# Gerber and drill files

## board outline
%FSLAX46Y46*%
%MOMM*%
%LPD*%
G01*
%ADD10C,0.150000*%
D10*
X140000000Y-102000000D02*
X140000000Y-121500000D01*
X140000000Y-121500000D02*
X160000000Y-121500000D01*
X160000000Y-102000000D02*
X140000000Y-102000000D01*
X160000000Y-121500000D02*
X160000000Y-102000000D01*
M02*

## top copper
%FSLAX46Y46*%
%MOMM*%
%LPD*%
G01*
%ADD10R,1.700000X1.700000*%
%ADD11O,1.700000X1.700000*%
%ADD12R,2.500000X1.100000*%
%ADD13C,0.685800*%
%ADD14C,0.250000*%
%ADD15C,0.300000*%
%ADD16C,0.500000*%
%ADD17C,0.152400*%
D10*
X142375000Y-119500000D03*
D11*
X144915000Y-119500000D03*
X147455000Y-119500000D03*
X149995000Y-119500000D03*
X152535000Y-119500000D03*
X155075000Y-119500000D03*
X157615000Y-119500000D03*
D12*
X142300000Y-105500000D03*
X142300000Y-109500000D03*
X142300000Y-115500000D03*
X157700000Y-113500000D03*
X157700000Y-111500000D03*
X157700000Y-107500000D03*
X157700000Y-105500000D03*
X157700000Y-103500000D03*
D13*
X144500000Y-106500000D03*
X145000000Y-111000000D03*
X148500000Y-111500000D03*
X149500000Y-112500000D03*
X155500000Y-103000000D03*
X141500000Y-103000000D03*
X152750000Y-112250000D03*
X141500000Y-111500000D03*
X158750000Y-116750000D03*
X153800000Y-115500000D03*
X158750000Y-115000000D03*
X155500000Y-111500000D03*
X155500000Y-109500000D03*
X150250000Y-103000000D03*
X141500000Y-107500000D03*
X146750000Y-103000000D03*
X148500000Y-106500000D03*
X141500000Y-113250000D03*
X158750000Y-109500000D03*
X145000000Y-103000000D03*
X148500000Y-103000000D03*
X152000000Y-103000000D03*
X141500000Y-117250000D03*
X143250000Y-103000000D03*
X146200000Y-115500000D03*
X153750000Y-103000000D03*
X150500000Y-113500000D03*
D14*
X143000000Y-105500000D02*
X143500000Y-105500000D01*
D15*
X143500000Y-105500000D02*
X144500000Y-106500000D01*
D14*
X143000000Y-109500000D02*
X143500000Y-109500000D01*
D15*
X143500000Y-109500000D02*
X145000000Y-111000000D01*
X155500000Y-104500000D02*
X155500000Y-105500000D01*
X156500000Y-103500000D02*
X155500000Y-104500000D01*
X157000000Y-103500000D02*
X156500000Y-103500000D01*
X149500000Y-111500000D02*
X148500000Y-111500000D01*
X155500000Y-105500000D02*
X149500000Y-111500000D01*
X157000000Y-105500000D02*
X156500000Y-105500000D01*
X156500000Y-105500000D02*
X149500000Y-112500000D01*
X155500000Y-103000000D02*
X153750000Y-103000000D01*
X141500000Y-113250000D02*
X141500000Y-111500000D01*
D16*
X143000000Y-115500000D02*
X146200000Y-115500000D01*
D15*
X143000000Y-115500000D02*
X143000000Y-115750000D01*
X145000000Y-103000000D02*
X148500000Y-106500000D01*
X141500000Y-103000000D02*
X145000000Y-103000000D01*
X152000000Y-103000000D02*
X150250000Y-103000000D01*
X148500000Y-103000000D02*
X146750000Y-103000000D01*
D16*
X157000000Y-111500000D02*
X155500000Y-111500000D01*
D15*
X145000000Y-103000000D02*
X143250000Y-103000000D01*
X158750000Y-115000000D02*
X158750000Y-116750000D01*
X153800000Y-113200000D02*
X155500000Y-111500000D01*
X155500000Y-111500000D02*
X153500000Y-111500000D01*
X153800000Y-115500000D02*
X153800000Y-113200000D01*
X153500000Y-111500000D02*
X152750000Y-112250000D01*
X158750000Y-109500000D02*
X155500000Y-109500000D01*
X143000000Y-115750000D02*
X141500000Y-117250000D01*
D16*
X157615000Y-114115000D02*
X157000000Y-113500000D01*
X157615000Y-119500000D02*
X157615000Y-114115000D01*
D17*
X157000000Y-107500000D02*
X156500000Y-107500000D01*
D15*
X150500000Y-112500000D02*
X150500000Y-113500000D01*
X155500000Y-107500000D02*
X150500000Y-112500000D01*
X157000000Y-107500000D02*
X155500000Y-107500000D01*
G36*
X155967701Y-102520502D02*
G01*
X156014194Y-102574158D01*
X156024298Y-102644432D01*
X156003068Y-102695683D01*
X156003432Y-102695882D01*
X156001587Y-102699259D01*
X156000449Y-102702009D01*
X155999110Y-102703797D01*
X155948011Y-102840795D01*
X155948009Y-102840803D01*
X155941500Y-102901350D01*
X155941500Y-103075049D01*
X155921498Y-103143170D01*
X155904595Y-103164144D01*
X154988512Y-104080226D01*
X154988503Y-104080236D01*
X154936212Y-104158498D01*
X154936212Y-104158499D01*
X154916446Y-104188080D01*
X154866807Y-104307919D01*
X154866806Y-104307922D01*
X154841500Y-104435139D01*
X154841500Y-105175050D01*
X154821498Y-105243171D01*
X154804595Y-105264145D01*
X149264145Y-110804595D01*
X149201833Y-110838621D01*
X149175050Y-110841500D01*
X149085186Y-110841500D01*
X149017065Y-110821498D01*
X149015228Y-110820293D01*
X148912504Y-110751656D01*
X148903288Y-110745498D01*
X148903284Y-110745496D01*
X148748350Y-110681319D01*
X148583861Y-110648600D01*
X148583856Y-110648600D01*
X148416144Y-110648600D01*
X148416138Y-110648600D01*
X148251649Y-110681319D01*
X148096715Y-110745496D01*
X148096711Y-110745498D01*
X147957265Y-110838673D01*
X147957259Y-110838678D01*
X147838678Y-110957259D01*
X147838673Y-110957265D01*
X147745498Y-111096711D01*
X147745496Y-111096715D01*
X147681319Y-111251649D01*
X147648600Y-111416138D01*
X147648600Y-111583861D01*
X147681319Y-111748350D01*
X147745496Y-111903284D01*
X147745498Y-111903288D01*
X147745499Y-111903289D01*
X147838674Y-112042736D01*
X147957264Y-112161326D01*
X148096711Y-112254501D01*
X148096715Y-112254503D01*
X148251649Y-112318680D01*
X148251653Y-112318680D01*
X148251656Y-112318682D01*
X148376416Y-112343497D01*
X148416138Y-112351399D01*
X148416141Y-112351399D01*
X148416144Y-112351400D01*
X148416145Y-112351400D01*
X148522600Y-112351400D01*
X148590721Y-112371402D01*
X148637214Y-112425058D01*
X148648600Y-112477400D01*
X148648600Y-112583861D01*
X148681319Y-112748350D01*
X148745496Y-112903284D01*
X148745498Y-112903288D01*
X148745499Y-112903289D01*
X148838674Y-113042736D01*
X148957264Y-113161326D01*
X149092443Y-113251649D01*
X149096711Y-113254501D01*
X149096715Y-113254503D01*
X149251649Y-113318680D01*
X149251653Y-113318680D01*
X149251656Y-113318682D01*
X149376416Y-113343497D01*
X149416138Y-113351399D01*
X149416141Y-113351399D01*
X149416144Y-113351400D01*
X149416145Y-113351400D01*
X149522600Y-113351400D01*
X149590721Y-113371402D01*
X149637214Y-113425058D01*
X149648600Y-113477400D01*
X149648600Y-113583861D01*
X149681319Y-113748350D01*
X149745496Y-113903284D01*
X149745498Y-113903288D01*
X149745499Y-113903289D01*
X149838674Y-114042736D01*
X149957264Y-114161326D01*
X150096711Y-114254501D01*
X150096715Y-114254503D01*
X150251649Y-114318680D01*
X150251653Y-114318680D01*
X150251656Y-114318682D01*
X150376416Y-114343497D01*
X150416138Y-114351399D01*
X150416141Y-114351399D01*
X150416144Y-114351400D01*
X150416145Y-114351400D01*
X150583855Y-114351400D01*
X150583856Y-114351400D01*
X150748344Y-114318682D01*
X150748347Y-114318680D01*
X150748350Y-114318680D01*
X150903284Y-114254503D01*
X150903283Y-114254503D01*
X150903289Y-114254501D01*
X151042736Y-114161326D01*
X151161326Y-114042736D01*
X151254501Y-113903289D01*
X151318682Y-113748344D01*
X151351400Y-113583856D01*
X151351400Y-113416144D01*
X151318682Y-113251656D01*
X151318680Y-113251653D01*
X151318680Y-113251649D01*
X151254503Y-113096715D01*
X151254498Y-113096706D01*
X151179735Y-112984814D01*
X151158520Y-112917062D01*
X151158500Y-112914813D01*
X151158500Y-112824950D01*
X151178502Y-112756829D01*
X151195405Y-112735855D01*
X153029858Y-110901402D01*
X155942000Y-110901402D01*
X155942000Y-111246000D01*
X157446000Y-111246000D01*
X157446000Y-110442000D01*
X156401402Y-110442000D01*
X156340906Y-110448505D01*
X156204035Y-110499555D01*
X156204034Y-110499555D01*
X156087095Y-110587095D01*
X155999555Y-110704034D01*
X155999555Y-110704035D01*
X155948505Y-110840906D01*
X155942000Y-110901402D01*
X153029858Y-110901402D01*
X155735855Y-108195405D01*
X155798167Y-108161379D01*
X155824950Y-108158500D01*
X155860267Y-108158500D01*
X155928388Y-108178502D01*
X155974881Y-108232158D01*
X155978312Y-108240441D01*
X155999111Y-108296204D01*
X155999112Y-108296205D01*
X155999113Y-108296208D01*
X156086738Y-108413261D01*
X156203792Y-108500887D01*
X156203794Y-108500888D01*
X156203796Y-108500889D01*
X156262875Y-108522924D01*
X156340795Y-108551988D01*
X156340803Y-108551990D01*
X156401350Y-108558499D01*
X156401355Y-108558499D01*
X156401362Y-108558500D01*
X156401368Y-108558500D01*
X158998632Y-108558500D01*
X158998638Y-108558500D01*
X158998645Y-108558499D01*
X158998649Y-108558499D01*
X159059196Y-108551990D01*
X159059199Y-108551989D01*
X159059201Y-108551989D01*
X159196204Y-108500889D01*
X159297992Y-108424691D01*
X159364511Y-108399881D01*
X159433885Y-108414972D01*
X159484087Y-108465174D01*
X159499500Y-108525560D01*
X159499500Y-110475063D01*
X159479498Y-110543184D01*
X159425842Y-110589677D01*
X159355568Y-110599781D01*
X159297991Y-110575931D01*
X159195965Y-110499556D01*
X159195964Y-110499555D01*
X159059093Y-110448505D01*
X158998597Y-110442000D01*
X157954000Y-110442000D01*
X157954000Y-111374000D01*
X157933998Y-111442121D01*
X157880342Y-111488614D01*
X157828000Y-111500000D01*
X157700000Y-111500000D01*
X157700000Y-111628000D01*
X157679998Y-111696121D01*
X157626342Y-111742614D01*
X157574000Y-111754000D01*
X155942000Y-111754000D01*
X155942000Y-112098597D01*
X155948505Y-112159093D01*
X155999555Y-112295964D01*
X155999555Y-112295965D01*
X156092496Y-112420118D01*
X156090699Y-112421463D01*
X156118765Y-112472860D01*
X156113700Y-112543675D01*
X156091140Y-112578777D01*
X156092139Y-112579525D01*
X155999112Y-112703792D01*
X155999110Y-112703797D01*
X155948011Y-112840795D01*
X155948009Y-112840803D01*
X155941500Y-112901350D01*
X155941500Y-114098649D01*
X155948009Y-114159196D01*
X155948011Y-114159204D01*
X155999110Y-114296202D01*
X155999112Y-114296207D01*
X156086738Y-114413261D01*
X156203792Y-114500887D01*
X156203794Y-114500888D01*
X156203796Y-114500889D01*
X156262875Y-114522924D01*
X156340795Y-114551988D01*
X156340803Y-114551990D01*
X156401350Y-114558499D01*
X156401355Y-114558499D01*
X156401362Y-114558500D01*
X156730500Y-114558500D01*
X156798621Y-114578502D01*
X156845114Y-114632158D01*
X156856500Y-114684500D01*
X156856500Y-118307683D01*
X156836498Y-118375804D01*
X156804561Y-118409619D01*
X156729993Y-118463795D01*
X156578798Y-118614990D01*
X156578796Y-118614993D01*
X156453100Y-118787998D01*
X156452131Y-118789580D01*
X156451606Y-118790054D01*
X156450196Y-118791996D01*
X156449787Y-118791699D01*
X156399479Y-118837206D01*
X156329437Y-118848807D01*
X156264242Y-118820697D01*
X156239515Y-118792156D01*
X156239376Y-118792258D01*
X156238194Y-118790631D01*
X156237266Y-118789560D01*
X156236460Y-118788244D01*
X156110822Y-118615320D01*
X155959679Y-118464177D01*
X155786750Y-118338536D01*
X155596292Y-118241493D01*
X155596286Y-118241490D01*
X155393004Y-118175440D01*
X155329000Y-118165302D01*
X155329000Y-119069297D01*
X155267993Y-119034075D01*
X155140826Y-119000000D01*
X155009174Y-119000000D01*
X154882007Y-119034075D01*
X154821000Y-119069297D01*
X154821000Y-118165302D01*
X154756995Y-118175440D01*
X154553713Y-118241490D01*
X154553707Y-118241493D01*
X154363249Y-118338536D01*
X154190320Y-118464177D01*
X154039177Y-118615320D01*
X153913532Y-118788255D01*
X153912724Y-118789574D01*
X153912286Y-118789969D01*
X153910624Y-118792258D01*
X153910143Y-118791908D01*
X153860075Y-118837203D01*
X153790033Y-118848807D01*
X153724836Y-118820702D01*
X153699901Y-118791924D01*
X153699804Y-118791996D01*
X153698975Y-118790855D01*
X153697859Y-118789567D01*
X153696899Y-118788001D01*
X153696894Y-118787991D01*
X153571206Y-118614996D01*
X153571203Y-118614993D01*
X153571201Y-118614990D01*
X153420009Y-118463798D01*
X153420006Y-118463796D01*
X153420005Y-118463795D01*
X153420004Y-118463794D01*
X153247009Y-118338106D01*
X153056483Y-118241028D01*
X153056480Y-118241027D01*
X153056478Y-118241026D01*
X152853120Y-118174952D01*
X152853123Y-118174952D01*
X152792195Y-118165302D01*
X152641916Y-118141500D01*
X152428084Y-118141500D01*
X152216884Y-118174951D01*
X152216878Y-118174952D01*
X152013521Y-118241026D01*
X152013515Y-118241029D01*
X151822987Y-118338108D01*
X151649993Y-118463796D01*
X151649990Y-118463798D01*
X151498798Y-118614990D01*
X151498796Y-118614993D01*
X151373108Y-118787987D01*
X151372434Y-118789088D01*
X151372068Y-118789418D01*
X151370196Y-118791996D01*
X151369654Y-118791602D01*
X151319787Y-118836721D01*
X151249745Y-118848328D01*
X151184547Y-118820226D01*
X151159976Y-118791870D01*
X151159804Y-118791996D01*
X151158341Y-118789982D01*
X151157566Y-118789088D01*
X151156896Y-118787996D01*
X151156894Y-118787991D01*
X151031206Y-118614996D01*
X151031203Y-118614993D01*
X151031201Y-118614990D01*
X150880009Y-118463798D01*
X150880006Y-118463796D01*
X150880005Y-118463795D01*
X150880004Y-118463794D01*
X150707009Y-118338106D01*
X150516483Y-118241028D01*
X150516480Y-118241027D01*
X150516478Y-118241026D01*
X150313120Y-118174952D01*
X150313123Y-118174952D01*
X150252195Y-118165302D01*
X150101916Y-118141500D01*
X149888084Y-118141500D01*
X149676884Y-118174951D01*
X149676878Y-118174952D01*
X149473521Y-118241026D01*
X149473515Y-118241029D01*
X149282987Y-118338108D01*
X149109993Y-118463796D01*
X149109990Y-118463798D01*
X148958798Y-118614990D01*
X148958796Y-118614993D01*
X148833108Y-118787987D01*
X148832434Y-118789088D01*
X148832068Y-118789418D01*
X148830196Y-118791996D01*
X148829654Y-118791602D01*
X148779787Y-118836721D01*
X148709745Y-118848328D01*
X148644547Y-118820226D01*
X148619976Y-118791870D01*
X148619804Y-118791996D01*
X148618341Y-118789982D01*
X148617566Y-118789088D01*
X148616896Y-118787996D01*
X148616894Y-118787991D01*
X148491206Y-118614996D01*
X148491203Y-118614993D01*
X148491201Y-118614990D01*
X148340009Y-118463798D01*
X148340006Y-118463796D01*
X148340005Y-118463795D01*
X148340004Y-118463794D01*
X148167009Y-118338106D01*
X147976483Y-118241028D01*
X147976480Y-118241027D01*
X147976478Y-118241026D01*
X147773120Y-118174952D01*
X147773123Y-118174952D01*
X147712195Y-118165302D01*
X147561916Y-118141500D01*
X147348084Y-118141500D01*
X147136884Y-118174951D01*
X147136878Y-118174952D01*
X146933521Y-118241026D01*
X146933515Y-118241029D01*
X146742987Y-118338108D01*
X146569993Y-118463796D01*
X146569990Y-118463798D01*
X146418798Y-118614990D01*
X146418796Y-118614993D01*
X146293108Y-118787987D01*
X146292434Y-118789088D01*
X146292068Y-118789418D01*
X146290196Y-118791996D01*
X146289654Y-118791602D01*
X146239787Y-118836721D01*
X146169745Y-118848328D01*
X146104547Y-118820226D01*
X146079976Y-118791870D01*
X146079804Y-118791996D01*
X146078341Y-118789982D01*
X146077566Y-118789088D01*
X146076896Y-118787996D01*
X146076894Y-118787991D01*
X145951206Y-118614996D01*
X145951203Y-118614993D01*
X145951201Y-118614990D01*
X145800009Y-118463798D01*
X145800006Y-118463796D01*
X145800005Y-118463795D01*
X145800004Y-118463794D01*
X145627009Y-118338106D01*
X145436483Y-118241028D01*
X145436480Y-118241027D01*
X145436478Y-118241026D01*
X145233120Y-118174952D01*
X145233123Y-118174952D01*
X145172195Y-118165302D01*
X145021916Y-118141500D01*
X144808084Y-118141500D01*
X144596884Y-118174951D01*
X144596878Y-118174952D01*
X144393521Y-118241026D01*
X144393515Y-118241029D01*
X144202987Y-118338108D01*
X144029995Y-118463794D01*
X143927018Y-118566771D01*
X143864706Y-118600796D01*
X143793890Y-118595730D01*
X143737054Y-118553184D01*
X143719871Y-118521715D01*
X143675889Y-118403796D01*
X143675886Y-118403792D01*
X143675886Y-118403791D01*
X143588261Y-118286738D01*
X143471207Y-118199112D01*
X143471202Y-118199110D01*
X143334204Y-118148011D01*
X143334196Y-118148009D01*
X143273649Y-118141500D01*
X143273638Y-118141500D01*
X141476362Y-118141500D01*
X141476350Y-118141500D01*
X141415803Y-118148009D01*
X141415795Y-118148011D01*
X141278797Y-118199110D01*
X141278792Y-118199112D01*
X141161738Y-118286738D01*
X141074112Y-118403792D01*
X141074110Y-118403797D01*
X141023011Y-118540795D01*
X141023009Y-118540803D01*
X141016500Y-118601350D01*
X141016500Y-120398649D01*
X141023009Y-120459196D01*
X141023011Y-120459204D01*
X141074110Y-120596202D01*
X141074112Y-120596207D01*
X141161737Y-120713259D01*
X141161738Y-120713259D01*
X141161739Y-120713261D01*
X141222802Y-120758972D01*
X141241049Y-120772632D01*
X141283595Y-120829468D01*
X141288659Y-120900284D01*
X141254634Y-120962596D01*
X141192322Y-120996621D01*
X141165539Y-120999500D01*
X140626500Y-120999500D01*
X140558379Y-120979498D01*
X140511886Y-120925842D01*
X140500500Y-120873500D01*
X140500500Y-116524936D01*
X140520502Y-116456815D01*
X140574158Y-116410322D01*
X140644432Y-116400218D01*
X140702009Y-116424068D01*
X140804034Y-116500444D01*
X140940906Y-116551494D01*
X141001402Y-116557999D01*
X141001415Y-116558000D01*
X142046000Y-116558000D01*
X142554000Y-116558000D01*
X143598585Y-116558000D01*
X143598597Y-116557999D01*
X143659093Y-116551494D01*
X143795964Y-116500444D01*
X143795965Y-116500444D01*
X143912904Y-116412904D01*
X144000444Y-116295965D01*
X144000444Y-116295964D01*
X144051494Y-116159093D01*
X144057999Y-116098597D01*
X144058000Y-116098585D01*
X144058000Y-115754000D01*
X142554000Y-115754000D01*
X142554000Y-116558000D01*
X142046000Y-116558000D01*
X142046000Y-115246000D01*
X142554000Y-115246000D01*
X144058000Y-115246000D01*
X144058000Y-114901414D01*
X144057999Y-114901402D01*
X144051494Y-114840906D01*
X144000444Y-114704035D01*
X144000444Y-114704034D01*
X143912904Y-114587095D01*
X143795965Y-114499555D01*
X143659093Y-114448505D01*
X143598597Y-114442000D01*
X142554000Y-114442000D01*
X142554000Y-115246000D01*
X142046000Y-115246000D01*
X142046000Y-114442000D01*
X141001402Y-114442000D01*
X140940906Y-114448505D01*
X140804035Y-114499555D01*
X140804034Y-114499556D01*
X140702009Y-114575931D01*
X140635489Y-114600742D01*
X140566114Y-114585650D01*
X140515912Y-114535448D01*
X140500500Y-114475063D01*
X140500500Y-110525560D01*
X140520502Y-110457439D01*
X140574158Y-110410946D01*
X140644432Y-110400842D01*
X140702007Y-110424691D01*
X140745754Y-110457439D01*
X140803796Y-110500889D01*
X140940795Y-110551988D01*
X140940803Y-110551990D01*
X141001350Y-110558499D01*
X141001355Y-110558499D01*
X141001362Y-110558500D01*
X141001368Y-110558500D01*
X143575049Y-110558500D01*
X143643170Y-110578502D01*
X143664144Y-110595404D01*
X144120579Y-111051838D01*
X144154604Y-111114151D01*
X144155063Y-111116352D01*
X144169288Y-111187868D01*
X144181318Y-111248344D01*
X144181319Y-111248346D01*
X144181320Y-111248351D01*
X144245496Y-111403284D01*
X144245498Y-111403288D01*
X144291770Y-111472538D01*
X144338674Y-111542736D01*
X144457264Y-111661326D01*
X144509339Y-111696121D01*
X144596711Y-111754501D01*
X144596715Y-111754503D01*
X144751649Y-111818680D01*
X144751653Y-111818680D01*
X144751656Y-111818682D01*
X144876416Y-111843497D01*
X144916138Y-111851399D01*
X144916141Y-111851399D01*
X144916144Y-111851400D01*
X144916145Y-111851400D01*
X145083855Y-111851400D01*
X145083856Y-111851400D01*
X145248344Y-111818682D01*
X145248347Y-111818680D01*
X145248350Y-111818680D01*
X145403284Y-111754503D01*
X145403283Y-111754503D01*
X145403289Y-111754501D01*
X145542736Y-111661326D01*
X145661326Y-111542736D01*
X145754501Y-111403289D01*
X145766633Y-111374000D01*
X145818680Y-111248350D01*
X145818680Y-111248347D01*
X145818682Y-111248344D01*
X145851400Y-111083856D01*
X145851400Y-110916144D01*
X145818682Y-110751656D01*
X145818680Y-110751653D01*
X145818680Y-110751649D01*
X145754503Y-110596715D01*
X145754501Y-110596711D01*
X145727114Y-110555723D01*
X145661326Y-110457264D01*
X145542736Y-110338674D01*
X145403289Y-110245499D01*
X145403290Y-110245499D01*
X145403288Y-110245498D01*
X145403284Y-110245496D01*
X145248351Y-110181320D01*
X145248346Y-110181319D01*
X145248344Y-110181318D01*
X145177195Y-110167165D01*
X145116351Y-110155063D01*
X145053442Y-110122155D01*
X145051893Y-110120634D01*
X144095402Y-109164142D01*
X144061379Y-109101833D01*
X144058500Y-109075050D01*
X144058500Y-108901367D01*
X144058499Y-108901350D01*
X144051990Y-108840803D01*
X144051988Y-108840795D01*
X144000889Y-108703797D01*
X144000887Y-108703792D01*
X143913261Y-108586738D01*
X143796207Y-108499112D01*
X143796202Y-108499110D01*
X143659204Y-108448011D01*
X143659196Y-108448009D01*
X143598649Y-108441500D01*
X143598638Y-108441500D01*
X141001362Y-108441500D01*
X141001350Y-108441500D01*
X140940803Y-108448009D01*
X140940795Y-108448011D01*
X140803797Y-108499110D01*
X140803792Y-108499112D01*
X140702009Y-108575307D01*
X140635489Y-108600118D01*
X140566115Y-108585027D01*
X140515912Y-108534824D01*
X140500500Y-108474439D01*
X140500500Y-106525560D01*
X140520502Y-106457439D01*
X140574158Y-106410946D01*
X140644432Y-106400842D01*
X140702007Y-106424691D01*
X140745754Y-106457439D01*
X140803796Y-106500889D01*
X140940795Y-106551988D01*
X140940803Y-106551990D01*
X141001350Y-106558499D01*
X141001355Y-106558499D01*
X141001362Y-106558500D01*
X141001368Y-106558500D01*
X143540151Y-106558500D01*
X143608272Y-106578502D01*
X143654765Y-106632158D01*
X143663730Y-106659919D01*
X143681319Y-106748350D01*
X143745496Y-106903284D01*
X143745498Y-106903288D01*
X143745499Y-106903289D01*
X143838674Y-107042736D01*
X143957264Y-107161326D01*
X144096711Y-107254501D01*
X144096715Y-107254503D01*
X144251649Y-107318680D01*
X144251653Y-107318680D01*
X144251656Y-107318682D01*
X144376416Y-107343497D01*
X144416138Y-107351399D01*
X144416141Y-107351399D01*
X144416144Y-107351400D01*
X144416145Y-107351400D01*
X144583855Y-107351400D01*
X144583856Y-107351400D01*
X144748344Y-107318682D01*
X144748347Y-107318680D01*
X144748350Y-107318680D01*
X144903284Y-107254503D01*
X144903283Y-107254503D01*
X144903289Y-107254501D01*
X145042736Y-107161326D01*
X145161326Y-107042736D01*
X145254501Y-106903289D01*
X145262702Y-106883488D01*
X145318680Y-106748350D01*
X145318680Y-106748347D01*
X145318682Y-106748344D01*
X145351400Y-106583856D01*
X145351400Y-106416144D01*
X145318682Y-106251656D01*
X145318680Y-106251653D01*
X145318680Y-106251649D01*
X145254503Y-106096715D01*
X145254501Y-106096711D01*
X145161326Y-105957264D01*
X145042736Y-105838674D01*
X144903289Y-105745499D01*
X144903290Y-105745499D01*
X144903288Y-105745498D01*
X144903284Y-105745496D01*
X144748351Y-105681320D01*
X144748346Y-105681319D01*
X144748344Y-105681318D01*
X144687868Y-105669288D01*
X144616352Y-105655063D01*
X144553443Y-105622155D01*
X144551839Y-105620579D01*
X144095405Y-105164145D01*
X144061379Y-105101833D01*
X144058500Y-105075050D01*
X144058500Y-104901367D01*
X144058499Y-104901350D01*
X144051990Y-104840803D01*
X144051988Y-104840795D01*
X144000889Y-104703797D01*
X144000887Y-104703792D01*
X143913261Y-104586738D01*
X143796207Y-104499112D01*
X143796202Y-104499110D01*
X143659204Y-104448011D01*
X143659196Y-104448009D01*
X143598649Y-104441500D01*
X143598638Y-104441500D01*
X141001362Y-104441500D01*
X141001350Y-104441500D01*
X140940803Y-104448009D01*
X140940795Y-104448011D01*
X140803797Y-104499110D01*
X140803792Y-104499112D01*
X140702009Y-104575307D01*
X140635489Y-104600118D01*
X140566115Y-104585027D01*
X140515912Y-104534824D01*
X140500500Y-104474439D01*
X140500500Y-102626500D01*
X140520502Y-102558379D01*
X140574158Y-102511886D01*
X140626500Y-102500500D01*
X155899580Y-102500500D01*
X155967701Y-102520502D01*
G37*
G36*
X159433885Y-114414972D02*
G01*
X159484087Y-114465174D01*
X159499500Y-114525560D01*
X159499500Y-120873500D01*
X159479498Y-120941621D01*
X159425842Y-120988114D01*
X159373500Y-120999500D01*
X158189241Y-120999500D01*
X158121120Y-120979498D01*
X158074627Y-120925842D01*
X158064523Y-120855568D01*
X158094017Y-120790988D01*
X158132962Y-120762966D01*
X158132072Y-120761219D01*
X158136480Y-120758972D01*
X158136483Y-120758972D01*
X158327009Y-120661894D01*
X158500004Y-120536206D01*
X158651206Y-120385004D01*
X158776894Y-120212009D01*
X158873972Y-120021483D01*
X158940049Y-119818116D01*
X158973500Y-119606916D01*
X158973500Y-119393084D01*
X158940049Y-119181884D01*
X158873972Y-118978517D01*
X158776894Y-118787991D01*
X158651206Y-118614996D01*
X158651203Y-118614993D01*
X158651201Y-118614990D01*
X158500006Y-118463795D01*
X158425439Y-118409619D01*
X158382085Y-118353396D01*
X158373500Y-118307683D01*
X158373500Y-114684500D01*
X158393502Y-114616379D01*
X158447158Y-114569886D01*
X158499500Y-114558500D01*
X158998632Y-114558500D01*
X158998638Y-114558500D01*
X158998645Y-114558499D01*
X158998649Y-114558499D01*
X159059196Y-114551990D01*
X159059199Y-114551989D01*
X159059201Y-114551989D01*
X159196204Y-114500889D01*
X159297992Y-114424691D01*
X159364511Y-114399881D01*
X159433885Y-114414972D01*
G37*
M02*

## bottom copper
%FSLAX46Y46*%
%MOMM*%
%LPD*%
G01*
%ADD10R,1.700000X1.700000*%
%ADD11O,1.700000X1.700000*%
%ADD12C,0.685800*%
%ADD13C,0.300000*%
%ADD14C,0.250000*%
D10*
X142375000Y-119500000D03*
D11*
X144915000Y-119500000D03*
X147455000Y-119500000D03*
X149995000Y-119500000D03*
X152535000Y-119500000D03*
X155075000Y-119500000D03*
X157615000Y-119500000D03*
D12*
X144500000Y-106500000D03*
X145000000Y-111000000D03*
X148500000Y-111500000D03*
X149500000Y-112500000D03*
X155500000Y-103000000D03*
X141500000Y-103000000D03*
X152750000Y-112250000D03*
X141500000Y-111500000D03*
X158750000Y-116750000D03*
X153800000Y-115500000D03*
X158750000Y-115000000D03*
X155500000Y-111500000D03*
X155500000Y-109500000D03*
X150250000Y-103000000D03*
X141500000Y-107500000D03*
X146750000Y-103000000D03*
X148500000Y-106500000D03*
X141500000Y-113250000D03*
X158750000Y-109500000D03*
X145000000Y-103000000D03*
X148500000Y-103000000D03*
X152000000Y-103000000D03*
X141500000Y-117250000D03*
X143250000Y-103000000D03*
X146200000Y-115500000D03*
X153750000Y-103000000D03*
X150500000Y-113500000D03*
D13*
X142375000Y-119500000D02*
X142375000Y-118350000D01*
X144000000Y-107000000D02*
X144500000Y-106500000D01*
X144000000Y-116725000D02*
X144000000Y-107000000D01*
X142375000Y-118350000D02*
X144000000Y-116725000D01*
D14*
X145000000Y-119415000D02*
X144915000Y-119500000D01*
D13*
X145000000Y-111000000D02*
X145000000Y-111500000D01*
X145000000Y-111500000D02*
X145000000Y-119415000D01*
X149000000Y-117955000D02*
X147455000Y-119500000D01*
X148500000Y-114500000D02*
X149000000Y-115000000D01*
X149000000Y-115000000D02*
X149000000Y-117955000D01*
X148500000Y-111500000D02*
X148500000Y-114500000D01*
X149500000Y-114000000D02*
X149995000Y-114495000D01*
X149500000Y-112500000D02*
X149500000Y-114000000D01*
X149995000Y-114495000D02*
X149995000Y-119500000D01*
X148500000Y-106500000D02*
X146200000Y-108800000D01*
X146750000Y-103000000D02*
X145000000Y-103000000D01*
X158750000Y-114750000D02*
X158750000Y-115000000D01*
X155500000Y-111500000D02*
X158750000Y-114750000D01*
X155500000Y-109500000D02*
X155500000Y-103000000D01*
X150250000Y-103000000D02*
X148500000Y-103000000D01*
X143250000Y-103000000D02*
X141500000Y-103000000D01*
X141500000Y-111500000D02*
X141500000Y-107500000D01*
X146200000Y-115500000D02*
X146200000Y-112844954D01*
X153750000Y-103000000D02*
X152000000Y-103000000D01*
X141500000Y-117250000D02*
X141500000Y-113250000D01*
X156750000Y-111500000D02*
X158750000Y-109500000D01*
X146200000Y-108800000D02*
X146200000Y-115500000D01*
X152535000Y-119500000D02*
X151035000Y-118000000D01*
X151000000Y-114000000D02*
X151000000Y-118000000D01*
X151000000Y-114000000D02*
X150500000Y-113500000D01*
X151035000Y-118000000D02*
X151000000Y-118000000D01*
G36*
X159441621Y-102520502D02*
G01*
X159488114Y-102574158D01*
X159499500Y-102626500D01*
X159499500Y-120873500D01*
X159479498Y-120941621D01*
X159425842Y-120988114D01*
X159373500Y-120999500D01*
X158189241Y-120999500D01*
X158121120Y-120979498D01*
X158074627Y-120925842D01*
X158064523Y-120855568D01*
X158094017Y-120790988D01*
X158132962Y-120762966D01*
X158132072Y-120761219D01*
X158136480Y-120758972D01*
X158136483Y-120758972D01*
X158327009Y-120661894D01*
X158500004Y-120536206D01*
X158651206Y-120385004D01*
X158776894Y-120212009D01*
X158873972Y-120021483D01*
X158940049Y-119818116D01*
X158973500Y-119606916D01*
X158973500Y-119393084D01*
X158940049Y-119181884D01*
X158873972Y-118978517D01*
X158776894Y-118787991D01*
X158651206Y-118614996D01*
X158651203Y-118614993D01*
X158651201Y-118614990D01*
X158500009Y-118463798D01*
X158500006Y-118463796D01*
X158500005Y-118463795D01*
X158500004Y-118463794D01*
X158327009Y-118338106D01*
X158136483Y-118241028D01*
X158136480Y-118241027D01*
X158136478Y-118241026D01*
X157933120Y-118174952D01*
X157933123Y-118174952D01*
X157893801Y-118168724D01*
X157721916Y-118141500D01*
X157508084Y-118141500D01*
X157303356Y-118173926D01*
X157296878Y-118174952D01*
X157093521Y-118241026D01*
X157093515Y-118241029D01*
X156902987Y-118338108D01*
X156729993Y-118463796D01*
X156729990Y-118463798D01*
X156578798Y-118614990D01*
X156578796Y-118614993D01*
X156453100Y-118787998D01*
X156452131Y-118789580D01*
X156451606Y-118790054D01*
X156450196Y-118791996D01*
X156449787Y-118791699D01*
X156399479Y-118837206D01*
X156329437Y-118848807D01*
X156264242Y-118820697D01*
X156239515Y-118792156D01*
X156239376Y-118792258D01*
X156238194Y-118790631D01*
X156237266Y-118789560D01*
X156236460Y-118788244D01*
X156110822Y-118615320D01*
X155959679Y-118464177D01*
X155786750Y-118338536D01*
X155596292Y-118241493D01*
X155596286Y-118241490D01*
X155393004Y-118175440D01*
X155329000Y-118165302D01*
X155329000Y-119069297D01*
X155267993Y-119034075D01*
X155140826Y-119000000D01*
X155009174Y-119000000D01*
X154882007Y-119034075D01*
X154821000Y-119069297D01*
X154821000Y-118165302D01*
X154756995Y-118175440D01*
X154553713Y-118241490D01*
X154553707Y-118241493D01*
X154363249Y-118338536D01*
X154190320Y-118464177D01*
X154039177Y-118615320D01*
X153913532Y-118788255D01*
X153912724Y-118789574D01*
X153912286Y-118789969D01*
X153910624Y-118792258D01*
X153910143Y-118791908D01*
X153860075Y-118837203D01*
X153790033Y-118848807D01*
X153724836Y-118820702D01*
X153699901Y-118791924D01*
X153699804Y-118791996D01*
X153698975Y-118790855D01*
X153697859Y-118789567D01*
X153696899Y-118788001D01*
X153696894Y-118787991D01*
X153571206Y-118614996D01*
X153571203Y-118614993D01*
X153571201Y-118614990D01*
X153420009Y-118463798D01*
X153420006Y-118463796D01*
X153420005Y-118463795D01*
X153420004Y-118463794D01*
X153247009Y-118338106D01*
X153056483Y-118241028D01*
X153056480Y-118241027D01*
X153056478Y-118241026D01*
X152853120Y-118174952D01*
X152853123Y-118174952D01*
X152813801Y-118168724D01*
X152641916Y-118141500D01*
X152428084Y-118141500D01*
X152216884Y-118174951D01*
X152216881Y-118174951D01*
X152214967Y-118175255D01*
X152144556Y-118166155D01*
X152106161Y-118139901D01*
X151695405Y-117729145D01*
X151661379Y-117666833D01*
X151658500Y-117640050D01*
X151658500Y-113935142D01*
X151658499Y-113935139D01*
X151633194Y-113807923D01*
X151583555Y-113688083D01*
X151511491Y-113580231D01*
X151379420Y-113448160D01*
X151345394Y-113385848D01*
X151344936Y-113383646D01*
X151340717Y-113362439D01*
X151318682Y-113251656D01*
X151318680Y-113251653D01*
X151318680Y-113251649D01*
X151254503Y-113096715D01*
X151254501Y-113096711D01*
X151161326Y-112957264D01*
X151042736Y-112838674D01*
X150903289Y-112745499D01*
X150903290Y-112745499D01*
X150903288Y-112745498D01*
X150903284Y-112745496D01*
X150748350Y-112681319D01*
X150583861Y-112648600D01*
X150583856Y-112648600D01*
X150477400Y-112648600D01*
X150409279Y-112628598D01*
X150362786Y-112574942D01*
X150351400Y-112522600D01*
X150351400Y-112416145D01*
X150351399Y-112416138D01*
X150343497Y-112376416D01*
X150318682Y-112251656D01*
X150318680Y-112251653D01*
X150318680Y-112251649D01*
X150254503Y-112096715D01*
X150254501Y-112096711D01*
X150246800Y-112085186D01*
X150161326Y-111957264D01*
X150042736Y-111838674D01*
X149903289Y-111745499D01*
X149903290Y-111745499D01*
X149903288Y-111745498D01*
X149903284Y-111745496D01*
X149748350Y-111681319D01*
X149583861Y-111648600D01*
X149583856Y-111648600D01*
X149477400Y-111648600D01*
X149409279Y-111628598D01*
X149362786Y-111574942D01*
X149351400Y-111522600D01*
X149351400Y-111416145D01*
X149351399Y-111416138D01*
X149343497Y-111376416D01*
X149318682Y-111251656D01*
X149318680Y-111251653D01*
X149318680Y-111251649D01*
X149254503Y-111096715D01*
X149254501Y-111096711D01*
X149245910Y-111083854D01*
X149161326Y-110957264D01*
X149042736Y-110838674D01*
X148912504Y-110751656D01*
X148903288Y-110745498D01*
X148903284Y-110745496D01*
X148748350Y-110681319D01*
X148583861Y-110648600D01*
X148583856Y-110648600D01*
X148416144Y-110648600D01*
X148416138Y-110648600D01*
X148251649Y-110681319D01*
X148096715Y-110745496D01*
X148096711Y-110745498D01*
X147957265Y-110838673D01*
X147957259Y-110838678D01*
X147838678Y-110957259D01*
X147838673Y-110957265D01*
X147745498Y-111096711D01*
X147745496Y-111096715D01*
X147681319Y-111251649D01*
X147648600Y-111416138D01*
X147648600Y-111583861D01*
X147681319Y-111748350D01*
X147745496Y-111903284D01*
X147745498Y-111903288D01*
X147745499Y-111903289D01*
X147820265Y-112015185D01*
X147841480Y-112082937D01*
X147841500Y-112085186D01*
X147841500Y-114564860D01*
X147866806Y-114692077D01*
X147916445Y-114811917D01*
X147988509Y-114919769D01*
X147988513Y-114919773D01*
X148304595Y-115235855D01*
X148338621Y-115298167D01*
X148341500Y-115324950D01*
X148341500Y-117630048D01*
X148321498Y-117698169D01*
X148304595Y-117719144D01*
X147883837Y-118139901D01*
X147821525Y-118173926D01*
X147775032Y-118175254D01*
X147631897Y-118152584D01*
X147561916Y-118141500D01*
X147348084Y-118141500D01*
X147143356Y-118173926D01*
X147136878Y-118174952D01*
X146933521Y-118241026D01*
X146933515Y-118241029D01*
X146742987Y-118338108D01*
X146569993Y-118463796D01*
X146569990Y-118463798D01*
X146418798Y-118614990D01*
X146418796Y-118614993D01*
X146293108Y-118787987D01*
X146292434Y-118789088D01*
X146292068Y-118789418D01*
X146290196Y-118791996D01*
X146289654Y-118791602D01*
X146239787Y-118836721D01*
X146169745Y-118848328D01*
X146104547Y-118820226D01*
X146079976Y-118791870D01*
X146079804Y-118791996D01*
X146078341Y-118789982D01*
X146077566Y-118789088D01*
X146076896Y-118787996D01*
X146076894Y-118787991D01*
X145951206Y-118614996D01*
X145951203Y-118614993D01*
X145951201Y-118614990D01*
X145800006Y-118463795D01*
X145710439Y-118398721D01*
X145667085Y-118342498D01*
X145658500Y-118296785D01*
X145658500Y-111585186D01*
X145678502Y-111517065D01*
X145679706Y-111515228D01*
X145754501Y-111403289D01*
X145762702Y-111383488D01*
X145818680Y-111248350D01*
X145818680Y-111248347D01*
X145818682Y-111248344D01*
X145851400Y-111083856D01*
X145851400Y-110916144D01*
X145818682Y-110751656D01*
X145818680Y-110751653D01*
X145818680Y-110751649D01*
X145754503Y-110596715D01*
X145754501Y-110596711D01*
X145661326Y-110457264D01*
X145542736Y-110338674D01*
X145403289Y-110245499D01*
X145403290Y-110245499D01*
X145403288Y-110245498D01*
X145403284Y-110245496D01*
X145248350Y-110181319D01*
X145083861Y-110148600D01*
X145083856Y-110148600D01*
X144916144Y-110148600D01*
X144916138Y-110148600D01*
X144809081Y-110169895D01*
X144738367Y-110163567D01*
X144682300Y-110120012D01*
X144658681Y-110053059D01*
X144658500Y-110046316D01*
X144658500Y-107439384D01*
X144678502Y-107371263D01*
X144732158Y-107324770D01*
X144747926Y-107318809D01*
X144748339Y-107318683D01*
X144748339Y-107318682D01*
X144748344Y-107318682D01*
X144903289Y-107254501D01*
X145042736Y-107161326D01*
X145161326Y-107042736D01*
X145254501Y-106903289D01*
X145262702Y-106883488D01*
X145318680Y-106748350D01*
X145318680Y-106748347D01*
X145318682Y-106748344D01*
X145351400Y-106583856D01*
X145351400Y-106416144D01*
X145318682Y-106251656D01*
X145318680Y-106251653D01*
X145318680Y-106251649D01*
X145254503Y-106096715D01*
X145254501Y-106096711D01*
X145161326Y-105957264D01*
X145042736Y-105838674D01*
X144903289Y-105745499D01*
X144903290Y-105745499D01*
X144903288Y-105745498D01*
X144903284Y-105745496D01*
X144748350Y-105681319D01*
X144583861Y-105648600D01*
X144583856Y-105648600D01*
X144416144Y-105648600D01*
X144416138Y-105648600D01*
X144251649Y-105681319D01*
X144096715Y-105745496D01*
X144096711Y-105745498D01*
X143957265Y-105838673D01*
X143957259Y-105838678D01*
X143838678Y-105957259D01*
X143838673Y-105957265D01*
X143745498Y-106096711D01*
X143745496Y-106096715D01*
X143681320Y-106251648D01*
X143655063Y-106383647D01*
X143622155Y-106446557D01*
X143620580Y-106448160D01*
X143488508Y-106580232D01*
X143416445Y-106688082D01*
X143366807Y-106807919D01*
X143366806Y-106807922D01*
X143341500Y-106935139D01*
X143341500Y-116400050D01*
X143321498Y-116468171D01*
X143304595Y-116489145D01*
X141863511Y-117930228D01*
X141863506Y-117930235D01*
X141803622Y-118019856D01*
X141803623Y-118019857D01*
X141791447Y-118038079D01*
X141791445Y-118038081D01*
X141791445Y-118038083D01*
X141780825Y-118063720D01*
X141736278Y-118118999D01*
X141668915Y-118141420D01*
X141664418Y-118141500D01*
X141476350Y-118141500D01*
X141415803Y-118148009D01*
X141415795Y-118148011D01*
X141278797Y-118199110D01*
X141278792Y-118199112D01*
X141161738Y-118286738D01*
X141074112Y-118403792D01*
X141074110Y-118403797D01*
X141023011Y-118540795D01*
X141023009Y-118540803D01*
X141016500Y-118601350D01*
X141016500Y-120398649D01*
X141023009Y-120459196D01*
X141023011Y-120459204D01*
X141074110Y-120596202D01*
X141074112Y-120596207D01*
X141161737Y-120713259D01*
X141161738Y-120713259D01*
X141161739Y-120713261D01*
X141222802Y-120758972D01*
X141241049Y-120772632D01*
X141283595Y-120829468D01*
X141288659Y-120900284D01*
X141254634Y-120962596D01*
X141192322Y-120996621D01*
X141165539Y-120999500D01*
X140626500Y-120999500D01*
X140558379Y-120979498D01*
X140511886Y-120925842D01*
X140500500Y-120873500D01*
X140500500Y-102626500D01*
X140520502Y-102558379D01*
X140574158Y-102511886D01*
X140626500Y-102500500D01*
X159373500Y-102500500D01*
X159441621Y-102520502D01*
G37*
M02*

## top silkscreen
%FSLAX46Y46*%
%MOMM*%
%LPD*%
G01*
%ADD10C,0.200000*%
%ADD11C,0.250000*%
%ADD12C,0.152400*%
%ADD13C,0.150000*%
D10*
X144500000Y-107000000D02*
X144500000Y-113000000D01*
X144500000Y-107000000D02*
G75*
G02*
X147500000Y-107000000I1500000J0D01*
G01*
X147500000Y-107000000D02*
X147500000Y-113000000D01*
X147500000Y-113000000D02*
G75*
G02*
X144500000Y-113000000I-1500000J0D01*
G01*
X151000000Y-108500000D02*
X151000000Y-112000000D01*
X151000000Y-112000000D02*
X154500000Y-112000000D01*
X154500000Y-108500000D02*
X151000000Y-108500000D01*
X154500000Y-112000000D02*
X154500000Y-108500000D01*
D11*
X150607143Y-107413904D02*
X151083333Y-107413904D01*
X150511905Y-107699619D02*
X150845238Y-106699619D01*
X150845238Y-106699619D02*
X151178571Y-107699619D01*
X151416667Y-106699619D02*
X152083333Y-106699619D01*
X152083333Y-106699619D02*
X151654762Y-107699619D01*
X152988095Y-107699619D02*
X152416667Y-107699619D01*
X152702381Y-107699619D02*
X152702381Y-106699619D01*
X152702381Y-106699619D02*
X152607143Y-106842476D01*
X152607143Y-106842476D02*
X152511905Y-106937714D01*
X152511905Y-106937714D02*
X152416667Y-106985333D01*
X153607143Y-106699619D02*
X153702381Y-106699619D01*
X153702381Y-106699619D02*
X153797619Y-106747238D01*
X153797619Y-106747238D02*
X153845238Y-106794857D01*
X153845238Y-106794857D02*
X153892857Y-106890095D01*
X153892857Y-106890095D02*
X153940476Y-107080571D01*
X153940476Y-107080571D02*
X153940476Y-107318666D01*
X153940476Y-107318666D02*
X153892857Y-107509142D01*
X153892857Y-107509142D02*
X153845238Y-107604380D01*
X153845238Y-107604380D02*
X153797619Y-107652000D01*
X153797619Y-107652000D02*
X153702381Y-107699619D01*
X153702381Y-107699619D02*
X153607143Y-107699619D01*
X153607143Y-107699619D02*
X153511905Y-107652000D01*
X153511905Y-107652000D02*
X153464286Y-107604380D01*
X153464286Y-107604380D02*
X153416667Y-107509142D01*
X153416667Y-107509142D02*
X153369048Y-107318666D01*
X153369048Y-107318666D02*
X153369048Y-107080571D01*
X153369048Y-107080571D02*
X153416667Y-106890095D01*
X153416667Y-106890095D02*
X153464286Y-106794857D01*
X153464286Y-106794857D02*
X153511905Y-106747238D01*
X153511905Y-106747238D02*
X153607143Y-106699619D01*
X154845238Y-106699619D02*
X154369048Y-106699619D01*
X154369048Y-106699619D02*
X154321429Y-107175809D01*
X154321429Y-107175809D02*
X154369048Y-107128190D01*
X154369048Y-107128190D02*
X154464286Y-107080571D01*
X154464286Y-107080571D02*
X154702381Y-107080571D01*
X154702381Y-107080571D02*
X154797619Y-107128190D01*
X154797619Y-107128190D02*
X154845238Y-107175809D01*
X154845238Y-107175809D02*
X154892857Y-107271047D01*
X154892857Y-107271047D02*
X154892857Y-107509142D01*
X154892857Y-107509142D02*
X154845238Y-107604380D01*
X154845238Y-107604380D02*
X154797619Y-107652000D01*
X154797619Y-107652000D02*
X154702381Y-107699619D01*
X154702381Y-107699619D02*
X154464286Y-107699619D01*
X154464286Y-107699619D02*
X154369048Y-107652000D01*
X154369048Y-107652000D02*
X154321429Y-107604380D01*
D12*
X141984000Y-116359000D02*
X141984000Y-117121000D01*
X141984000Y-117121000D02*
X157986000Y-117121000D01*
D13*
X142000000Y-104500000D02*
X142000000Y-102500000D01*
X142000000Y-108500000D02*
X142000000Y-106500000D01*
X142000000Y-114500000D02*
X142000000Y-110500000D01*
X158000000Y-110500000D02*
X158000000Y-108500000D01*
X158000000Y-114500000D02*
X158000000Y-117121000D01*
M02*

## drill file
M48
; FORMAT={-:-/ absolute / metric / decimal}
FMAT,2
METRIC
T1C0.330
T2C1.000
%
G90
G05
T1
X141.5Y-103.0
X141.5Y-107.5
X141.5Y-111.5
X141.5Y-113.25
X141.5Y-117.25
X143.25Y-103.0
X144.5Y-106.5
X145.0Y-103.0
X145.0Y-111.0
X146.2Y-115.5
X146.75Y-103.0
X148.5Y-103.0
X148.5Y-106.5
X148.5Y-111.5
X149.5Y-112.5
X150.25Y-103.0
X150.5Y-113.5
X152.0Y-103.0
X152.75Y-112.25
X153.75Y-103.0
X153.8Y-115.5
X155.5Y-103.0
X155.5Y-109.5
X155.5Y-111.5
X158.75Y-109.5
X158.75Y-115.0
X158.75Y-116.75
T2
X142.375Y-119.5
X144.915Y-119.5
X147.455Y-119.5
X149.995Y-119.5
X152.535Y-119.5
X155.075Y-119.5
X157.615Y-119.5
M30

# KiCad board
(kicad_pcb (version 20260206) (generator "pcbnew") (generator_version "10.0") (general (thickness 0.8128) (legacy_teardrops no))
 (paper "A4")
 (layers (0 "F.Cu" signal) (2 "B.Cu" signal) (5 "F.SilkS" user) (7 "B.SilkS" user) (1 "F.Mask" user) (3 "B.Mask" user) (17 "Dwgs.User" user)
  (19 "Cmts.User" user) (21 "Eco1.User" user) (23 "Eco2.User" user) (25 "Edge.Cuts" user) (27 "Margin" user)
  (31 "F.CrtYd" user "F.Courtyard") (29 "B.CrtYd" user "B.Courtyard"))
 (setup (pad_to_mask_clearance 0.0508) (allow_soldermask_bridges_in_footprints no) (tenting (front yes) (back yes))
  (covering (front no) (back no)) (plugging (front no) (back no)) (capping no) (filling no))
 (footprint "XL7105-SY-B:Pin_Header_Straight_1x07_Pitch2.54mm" (layer "F.Cu") (at 142.375 119.5 90)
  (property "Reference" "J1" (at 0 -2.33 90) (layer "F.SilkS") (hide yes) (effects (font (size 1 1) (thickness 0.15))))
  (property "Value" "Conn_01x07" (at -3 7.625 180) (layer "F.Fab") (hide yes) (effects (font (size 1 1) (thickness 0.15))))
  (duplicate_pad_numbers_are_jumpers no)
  (pad "1" thru_hole rect (at 0 0 90) (size 1.7 1.7) (drill 1) (layers "*.Cu" "*.Mask") (remove_unused_layers no) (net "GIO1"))
  (pad "2" thru_hole oval (at 0 2.54 90) (size 1.7 1.7) (drill 1) (layers "*.Cu" "*.Mask") (remove_unused_layers no) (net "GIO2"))
  (pad "3" thru_hole oval (at 0 5.08 90) (size 1.7 1.7) (drill 1) (layers "*.Cu" "*.Mask") (remove_unused_layers no) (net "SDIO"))
  (pad "4" thru_hole oval (at 0 7.62 90) (size 1.7 1.7) (drill 1) (layers "*.Cu" "*.Mask") (remove_unused_layers no) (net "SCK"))
  (pad "5" thru_hole oval (at 0 10.16 90) (size 1.7 1.7) (drill 1) (layers "*.Cu" "*.Mask") (remove_unused_layers no) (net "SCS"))
  (pad "6" thru_hole oval (at 0 12.7 90) (size 1.7 1.7) (drill 1) (layers "*.Cu" "*.Mask") (remove_unused_layers no) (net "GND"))
  (pad "7" thru_hole oval (at 0 15.24 90) (size 1.7 1.7) (drill 1) (layers "*.Cu" "*.Mask") (remove_unused_layers no) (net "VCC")))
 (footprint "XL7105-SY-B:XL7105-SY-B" (layer "F.Cu") (at 143 103.5)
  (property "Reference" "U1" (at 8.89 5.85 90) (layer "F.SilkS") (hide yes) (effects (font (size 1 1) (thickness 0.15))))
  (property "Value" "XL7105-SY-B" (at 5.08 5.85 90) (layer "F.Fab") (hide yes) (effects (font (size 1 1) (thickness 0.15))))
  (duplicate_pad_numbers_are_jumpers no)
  (fp_line (start -1.016 12.859) (end -1.016 13.621) (stroke (width 0.1524) (type solid)) (layer "F.SilkS"))
  (fp_line (start -1.016 13.621) (end 14.986 13.621) (stroke (width 0.1524) (type solid)) (layer "F.SilkS"))
  (fp_line (start -1 1) (end -1 -1) (stroke (width 0.15) (type solid)) (layer "F.SilkS"))
  (fp_line (start -1 5) (end -1 3) (stroke (width 0.15) (type solid)) (layer "F.SilkS"))
  (fp_line (start -1 11) (end -1 7) (stroke (width 0.15) (type solid)) (layer "F.SilkS"))
  (fp_line (start 15 7) (end 15 5) (stroke (width 0.15) (type solid)) (layer "F.SilkS"))
  (fp_line (start 15 11) (end 15 13.621) (stroke (width 0.15) (type solid)) (layer "F.SilkS"))
  (pad "2" smd rect (at 0 2) (size 2.5 1.1) (drill (offset -0.7 0)) (layers "F.Cu" "F.Mask") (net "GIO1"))
  (pad "4" smd rect (at 0 6) (size 2.5 1.1) (drill (offset -0.7 0)) (layers "F.Cu" "F.Mask") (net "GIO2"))
  (pad "7" smd rect (at 0 12) (size 2.5 1.1) (drill (offset -0.7 0)) (layers "F.Cu" "F.Mask") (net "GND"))
  (pad "9" smd rect (at 14 10) (size 2.5 1.1) (drill (offset 0.7 0)) (layers "F.Cu" "F.Mask") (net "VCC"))
  (pad "10" smd rect (at 14 8) (size 2.5 1.1) (drill (offset 0.7 0)) (layers "F.Cu" "F.Mask") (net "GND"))
  (pad "12" smd rect (at 14 4) (size 2.5 1.1) (drill (offset 0.7 0)) (layers "F.Cu" "F.Mask") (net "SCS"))
  (pad "13" smd rect (at 14 2) (size 2.5 1.1) (drill (offset 0.7 0)) (layers "F.Cu" "F.Mask") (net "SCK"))
  (pad "14" smd rect (at 14 0) (size 2.5 1.1) (drill (offset 0.7 0)) (layers "F.Cu" "F.Mask") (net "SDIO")))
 (gr_line (start 144.5 107) (end 144.5 113) (stroke (width 0.2) (type solid)) (layer "F.SilkS"))
 (gr_arc (start 144.5 107) (mid 146 105.5) (end 147.5 107) (stroke (width 0.2) (type solid)) (layer "F.SilkS"))
 (gr_line (start 147.5 107) (end 147.5 113) (stroke (width 0.2) (type solid)) (layer "F.SilkS"))
 (gr_arc (start 147.5 113) (mid 146 114.5) (end 144.5 113) (stroke (width 0.2) (type solid)) (layer "F.SilkS"))
 (gr_line (start 151 108.5) (end 151 112) (stroke (width 0.2) (type solid)) (layer "F.SilkS"))
 (gr_line (start 151 112) (end 154.5 112) (stroke (width 0.2) (type solid)) (layer "F.SilkS"))
 (gr_line (start 154.5 108.5) (end 151 108.5) (stroke (width 0.2) (type solid)) (layer "F.SilkS"))
 (gr_line (start 154.5 112) (end 154.5 108.5) (stroke (width 0.2) (type solid)) (layer "F.SilkS"))
 (gr_line (start 140 102) (end 140 121.5) (stroke (width 0.15) (type solid)) (layer "Edge.Cuts"))
 (gr_line (start 140 121.5) (end 160 121.5) (stroke (width 0.15) (type solid)) (layer "Edge.Cuts"))
 (gr_line (start 160 102) (end 140 102) (stroke (width 0.15) (type solid)) (layer "Edge.Cuts"))
 (gr_line (start 160 121.5) (end 160 102) (stroke (width 0.15) (type solid)) (layer "Edge.Cuts"))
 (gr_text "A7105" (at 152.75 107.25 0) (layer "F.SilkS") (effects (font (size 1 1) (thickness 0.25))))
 (segment (start 143 105.5) (end 143.5 105.5) (width 0.25) (layer "F.Cu") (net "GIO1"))
 (segment (start 143.5 105.5) (end 144.5 106.5) (width 0.3) (layer "F.Cu") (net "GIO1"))
 (via (at 144.5 106.5) (size 0.6858) (drill 0.3302) (layers "F.Cu" "B.Cu") (capping no) (covering (front no) (back no))
  (plugging (front no) (back no)) (filling no) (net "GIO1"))
 (segment (start 142.375 119.5) (end 142.375 118.35) (width 0.3) (layer "B.Cu") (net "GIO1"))
 (segment (start 144 107) (end 144.5 106.5) (width 0.3) (layer "B.Cu") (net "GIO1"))
 (segment (start 144 116.725) (end 144 107) (width 0.3) (layer "B.Cu") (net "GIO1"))
 (segment (start 142.375 118.35) (end 144 116.725) (width 0.3) (layer "B.Cu") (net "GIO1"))
 (segment (start 143 109.5) (end 143.5 109.5) (width 0.25) (layer "F.Cu") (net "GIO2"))
 (segment (start 143.5 109.5) (end 145 111) (width 0.3) (layer "F.Cu") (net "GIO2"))
 (via (at 145 111) (size 0.6858) (drill 0.3302) (layers "F.Cu" "B.Cu") (capping no) (covering (front no) (back no))
  (plugging (front no) (back no)) (filling no) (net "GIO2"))
 (segment (start 145 119.415) (end 144.915 119.5) (width 0.25) (layer "B.Cu") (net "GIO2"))
 (segment (start 145 111) (end 145 111.5) (width 0.3) (layer "B.Cu") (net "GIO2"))
 (segment (start 145 111.5) (end 145 119.415) (width 0.3) (layer "B.Cu") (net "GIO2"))
 (segment (start 155.5 104.5) (end 155.5 105.5) (width 0.3) (layer "F.Cu") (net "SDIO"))
 (segment (start 156.5 103.5) (end 155.5 104.5) (width 0.3) (layer "F.Cu") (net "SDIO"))
 (segment (start 157 103.5) (end 156.5 103.5) (width 0.3) (layer "F.Cu") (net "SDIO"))
 (segment (start 149.5 111.5) (end 148.5 111.5) (width 0.3) (layer "F.Cu") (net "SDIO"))
 (segment (start 155.5 105.5) (end 149.5 111.5) (width 0.3) (layer "F.Cu") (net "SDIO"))
 (via (at 148.5 111.5) (size 0.6858) (drill 0.3302) (layers "F.Cu" "B.Cu") (capping no) (covering (front no) (back no))
  (plugging (front no) (back no)) (filling no) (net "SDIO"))
 (segment (start 149 117.955) (end 147.455 119.5) (width 0.3) (layer "B.Cu") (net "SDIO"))
 (segment (start 148.5 114.5) (end 149 115) (width 0.3) (layer "B.Cu") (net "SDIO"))
 (segment (start 149 115) (end 149 117.955) (width 0.3) (layer "B.Cu") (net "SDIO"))
 (segment (start 148.5 111.5) (end 148.5 114.5) (width 0.3) (layer "B.Cu") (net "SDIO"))
 (segment (start 157 105.5) (end 156.5 105.5) (width 0.3) (layer "F.Cu") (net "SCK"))
 (segment (start 156.5 105.5) (end 149.5 112.5) (width 0.3) (layer "F.Cu") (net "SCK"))
 (via (at 149.5 112.5) (size 0.6858) (drill 0.3302) (layers "F.Cu" "B.Cu") (capping no) (covering (front no) (back no))
  (plugging (front no) (back no)) (filling no) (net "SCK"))
 (segment (start 149.5 114) (end 149.995 114.495) (width 0.3) (layer "B.Cu") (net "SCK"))
 (segment (start 149.5 112.5) (end 149.5 114) (width 0.3) (layer "B.Cu") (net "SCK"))
 (segment (start 149.995 114.495) (end 149.995 119.5) (width 0.3) (layer "B.Cu") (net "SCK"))
 (segment (start 155.5 103) (end 153.75 103) (width 0.3) (layer "F.Cu") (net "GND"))
 (segment (start 141.5 113.25) (end 141.5 111.5) (width 0.3) (layer "F.Cu") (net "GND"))
 (segment (start 143 115.5) (end 146.2 115.5) (width 0.5) (layer "F.Cu") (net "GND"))
 (segment (start 143 115.5) (end 143 115.75) (width 0.3) (layer "F.Cu") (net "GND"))
 (segment (start 145 103) (end 148.5 106.5) (width 0.3) (layer "F.Cu") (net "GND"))
 (segment (start 141.5 103) (end 145 103) (width 0.3) (layer "F.Cu") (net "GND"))
 (segment (start 152 103) (end 150.25 103) (width 0.3) (layer "F.Cu") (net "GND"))
 (segment (start 148.5 103) (end 146.75 103) (width 0.3) (layer "F.Cu") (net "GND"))
 (segment (start 157 111.5) (end 155.5 111.5) (width 0.5) (layer "F.Cu") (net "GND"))
 (segment (start 145 103) (end 143.25 103) (width 0.3) (layer "F.Cu") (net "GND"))
 (segment (start 158.75 115) (end 158.75 116.75) (width 0.3) (layer "F.Cu") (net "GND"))
 (segment (start 153.8 113.2) (end 155.5 111.5) (width 0.3) (layer "F.Cu") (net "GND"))
 (segment (start 155.5 111.5) (end 153.5 111.5) (width 0.3) (layer "F.Cu") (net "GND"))
 (segment (start 153.8 115.5) (end 153.8 113.2) (width 0.3) (layer "F.Cu") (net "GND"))
 (segment (start 153.5 111.5) (end 152.75 112.25) (width 0.3) (layer "F.Cu") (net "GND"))
 (segment (start 158.75 109.5) (end 155.5 109.5) (width 0.3) (layer "F.Cu") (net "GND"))
 (segment (start 143 115.75) (end 141.5 117.25) (width 0.3) (layer "F.Cu") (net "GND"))
 (via (at 155.5 103) (size 0.6858) (drill 0.3302) (layers "F.Cu" "B.Cu") (capping no) (covering (front no) (back no))
  (plugging (front no) (back no)) (filling no) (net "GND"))
 (via (at 141.5 103) (size 0.6858) (drill 0.3302) (layers "F.Cu" "B.Cu") (capping no) (covering (front no) (back no))
  (plugging (front no) (back no)) (filling no) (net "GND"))
 (via (at 152.75 112.25) (size 0.6858) (drill 0.3302) (layers "F.Cu" "B.Cu") (capping no) (covering (front no) (back no))
  (plugging (front no) (back no)) (filling no) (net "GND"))
 (via (at 141.5 111.5) (size 0.6858) (drill 0.3302) (layers "F.Cu" "B.Cu") (capping no) (covering (front no) (back no))
  (plugging (front no) (back no)) (filling no) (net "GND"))
 (via (at 158.75 116.75) (size 0.6858) (drill 0.3302) (layers "F.Cu" "B.Cu") (capping no) (covering (front no) (back no))
  (plugging (front no) (back no)) (filling no) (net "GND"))
 (via (at 153.8 115.5) (size 0.6858) (drill 0.3302) (layers "F.Cu" "B.Cu") (capping no) (covering (front no) (back no))
  (plugging (front no) (back no)) (filling no) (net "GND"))
 (via (at 158.75 115) (size 0.6858) (drill 0.3302) (layers "F.Cu" "B.Cu") (capping no) (covering (front no) (back no))
  (plugging (front no) (back no)) (filling no) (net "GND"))
 (via (at 155.5 111.5) (size 0.6858) (drill 0.3302) (layers "F.Cu" "B.Cu") (capping no) (covering (front no) (back no))
  (plugging (front no) (back no)) (filling no) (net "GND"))
 (via (at 155.5 109.5) (size 0.6858) (drill 0.3302) (layers "F.Cu" "B.Cu") (capping no) (covering (front no) (back no))
  (plugging (front no) (back no)) (filling no) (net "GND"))
 (via (at 150.25 103) (size 0.6858) (drill 0.3302) (layers "F.Cu" "B.Cu") (capping no) (covering (front no) (back no))
  (plugging (front no) (back no)) (filling no) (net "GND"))
 (via (at 141.5 107.5) (size 0.6858) (drill 0.3302) (layers "F.Cu" "B.Cu") (capping no) (covering (front no) (back no))
  (plugging (front no) (back no)) (filling no) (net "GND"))
 (via (at 146.75 103) (size 0.6858) (drill 0.3302) (layers "F.Cu" "B.Cu") (capping no) (covering (front no) (back no))
  (plugging (front no) (back no)) (filling no) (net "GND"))
 (via (at 148.5 106.5) (size 0.6858) (drill 0.3302) (layers "F.Cu" "B.Cu") (capping no) (covering (front no) (back no))
  (plugging (front no) (back no)) (filling no) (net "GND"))
 (via (at 141.5 113.25) (size 0.6858) (drill 0.3302) (layers "F.Cu" "B.Cu") (capping no) (covering (front no) (back no))
  (plugging (front no) (back no)) (filling no) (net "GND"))
 (via (at 158.75 109.5) (size 0.6858) (drill 0.3302) (layers "F.Cu" "B.Cu") (capping no) (covering (front no) (back no))
  (plugging (front no) (back no)) (filling no) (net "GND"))
 (via (at 145 103) (size 0.6858) (drill 0.3302) (layers "F.Cu" "B.Cu") (capping no) (covering (front no) (back no))
  (plugging (front no) (back no)) (filling no) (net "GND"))
 (via (at 148.5 103) (size 0.6858) (drill 0.3302) (layers "F.Cu" "B.Cu") (capping no) (covering (front no) (back no))
  (plugging (front no) (back no)) (filling no) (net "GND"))
 (via (at 152 103) (size 0.6858) (drill 0.3302) (layers "F.Cu" "B.Cu") (capping no) (covering (front no) (back no))
  (plugging (front no) (back no)) (filling no) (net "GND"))
 (via (at 141.5 117.25) (size 0.6858) (drill 0.3302) (layers "F.Cu" "B.Cu") (capping no) (covering (front no) (back no))
  (plugging (front no) (back no)) (filling no) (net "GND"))
 (via (at 143.25 103) (size 0.6858) (drill 0.3302) (layers "F.Cu" "B.Cu") (capping no) (covering (front no) (back no))
  (plugging (front no) (back no)) (filling no) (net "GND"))
 (via (at 146.2 115.5) (size 0.6858) (drill 0.3302) (layers "F.Cu" "B.Cu") (capping no) (covering (front no) (back no))
  (plugging (front no) (back no)) (filling no) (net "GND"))
 (via (at 153.75 103) (size 0.6858) (drill 0.3302) (layers "F.Cu" "B.Cu") (capping no) (covering (front no) (back no))
  (plugging (front no) (back no)) (filling no) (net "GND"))
 (segment (start 148.5 106.5) (end 146.2 108.8) (width 0.3) (layer "B.Cu") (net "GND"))
 (segment (start 146.75 103) (end 145 103) (width 0.3) (layer "B.Cu") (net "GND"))
 (segment (start 158.75 114.75) (end 158.75 115) (width 0.3) (layer "B.Cu") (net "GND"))
 (segment (start 155.5 111.5) (end 158.75 114.75) (width 0.3) (layer "B.Cu") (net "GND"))
 (segment (start 155.5 109.5) (end 155.5 103) (width 0.3) (layer "B.Cu") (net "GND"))
 (segment (start 150.25 103) (end 148.5 103) (width 0.3) (layer "B.Cu") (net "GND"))
 (segment (start 143.25 103) (end 141.5 103) (width 0.3) (layer "B.Cu") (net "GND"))
 (segment (start 141.5 111.5) (end 141.5 107.5) (width 0.3) (layer "B.Cu") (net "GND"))
 (segment (start 146.2 115.5) (end 146.2 112.844954) (width 0.3) (layer "B.Cu") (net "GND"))
 (segment (start 153.75 103) (end 152 103) (width 0.3) (layer "B.Cu") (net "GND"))
 (segment (start 141.5 117.25) (end 141.5 113.25) (width 0.3) (layer "B.Cu") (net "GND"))
 (segment (start 156.75 111.5) (end 158.75 109.5) (width 0.3) (layer "B.Cu") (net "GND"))
 (segment (start 146.2 108.8) (end 146.2 115.5) (width 0.3) (layer "B.Cu") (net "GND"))
 (segment (start 157.615 114.115) (end 157 113.5) (width 0.5) (layer "F.Cu") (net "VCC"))
 (segment (start 157.615 119.5) (end 157.615 114.115) (width 0.5) (layer "F.Cu") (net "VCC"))
 (segment (start 157 107.5) (end 156.5 107.5) (width 0.1524) (layer "F.Cu") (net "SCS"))
 (segment (start 150.5 112.5) (end 150.5 113.5) (width 0.3) (layer "F.Cu") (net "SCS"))
 (segment (start 155.5 107.5) (end 150.5 112.5) (width 0.3) (layer "F.Cu") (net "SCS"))
 (segment (start 157 107.5) (end 155.5 107.5) (width 0.3) (layer "F.Cu") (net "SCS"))
 (via (at 150.5 113.5) (size 0.6858) (drill 0.3302) (layers "F.Cu" "B.Cu") (capping no) (covering (front no) (back no))
  (plugging (front no) (back no)) (filling no) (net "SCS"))
 (segment (start 152.535 119.5) (end 151.035 118) (width 0.3) (layer "B.Cu") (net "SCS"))
 (segment (start 151 114) (end 151 118) (width 0.3) (layer "B.Cu") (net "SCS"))
 (segment (start 151 114) (end 150.5 113.5) (width 0.3) (layer "B.Cu") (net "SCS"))
 (segment (start 151.035 118) (end 151 118) (width 0.3) (layer "B.Cu") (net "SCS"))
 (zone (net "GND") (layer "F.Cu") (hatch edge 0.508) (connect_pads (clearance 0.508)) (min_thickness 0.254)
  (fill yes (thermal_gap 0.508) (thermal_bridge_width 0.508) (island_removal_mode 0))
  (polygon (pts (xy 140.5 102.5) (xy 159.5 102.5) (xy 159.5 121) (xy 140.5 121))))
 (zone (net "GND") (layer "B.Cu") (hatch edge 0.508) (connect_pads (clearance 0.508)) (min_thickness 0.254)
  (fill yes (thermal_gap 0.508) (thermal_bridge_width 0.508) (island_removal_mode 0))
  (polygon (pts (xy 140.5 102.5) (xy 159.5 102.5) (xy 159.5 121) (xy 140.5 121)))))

